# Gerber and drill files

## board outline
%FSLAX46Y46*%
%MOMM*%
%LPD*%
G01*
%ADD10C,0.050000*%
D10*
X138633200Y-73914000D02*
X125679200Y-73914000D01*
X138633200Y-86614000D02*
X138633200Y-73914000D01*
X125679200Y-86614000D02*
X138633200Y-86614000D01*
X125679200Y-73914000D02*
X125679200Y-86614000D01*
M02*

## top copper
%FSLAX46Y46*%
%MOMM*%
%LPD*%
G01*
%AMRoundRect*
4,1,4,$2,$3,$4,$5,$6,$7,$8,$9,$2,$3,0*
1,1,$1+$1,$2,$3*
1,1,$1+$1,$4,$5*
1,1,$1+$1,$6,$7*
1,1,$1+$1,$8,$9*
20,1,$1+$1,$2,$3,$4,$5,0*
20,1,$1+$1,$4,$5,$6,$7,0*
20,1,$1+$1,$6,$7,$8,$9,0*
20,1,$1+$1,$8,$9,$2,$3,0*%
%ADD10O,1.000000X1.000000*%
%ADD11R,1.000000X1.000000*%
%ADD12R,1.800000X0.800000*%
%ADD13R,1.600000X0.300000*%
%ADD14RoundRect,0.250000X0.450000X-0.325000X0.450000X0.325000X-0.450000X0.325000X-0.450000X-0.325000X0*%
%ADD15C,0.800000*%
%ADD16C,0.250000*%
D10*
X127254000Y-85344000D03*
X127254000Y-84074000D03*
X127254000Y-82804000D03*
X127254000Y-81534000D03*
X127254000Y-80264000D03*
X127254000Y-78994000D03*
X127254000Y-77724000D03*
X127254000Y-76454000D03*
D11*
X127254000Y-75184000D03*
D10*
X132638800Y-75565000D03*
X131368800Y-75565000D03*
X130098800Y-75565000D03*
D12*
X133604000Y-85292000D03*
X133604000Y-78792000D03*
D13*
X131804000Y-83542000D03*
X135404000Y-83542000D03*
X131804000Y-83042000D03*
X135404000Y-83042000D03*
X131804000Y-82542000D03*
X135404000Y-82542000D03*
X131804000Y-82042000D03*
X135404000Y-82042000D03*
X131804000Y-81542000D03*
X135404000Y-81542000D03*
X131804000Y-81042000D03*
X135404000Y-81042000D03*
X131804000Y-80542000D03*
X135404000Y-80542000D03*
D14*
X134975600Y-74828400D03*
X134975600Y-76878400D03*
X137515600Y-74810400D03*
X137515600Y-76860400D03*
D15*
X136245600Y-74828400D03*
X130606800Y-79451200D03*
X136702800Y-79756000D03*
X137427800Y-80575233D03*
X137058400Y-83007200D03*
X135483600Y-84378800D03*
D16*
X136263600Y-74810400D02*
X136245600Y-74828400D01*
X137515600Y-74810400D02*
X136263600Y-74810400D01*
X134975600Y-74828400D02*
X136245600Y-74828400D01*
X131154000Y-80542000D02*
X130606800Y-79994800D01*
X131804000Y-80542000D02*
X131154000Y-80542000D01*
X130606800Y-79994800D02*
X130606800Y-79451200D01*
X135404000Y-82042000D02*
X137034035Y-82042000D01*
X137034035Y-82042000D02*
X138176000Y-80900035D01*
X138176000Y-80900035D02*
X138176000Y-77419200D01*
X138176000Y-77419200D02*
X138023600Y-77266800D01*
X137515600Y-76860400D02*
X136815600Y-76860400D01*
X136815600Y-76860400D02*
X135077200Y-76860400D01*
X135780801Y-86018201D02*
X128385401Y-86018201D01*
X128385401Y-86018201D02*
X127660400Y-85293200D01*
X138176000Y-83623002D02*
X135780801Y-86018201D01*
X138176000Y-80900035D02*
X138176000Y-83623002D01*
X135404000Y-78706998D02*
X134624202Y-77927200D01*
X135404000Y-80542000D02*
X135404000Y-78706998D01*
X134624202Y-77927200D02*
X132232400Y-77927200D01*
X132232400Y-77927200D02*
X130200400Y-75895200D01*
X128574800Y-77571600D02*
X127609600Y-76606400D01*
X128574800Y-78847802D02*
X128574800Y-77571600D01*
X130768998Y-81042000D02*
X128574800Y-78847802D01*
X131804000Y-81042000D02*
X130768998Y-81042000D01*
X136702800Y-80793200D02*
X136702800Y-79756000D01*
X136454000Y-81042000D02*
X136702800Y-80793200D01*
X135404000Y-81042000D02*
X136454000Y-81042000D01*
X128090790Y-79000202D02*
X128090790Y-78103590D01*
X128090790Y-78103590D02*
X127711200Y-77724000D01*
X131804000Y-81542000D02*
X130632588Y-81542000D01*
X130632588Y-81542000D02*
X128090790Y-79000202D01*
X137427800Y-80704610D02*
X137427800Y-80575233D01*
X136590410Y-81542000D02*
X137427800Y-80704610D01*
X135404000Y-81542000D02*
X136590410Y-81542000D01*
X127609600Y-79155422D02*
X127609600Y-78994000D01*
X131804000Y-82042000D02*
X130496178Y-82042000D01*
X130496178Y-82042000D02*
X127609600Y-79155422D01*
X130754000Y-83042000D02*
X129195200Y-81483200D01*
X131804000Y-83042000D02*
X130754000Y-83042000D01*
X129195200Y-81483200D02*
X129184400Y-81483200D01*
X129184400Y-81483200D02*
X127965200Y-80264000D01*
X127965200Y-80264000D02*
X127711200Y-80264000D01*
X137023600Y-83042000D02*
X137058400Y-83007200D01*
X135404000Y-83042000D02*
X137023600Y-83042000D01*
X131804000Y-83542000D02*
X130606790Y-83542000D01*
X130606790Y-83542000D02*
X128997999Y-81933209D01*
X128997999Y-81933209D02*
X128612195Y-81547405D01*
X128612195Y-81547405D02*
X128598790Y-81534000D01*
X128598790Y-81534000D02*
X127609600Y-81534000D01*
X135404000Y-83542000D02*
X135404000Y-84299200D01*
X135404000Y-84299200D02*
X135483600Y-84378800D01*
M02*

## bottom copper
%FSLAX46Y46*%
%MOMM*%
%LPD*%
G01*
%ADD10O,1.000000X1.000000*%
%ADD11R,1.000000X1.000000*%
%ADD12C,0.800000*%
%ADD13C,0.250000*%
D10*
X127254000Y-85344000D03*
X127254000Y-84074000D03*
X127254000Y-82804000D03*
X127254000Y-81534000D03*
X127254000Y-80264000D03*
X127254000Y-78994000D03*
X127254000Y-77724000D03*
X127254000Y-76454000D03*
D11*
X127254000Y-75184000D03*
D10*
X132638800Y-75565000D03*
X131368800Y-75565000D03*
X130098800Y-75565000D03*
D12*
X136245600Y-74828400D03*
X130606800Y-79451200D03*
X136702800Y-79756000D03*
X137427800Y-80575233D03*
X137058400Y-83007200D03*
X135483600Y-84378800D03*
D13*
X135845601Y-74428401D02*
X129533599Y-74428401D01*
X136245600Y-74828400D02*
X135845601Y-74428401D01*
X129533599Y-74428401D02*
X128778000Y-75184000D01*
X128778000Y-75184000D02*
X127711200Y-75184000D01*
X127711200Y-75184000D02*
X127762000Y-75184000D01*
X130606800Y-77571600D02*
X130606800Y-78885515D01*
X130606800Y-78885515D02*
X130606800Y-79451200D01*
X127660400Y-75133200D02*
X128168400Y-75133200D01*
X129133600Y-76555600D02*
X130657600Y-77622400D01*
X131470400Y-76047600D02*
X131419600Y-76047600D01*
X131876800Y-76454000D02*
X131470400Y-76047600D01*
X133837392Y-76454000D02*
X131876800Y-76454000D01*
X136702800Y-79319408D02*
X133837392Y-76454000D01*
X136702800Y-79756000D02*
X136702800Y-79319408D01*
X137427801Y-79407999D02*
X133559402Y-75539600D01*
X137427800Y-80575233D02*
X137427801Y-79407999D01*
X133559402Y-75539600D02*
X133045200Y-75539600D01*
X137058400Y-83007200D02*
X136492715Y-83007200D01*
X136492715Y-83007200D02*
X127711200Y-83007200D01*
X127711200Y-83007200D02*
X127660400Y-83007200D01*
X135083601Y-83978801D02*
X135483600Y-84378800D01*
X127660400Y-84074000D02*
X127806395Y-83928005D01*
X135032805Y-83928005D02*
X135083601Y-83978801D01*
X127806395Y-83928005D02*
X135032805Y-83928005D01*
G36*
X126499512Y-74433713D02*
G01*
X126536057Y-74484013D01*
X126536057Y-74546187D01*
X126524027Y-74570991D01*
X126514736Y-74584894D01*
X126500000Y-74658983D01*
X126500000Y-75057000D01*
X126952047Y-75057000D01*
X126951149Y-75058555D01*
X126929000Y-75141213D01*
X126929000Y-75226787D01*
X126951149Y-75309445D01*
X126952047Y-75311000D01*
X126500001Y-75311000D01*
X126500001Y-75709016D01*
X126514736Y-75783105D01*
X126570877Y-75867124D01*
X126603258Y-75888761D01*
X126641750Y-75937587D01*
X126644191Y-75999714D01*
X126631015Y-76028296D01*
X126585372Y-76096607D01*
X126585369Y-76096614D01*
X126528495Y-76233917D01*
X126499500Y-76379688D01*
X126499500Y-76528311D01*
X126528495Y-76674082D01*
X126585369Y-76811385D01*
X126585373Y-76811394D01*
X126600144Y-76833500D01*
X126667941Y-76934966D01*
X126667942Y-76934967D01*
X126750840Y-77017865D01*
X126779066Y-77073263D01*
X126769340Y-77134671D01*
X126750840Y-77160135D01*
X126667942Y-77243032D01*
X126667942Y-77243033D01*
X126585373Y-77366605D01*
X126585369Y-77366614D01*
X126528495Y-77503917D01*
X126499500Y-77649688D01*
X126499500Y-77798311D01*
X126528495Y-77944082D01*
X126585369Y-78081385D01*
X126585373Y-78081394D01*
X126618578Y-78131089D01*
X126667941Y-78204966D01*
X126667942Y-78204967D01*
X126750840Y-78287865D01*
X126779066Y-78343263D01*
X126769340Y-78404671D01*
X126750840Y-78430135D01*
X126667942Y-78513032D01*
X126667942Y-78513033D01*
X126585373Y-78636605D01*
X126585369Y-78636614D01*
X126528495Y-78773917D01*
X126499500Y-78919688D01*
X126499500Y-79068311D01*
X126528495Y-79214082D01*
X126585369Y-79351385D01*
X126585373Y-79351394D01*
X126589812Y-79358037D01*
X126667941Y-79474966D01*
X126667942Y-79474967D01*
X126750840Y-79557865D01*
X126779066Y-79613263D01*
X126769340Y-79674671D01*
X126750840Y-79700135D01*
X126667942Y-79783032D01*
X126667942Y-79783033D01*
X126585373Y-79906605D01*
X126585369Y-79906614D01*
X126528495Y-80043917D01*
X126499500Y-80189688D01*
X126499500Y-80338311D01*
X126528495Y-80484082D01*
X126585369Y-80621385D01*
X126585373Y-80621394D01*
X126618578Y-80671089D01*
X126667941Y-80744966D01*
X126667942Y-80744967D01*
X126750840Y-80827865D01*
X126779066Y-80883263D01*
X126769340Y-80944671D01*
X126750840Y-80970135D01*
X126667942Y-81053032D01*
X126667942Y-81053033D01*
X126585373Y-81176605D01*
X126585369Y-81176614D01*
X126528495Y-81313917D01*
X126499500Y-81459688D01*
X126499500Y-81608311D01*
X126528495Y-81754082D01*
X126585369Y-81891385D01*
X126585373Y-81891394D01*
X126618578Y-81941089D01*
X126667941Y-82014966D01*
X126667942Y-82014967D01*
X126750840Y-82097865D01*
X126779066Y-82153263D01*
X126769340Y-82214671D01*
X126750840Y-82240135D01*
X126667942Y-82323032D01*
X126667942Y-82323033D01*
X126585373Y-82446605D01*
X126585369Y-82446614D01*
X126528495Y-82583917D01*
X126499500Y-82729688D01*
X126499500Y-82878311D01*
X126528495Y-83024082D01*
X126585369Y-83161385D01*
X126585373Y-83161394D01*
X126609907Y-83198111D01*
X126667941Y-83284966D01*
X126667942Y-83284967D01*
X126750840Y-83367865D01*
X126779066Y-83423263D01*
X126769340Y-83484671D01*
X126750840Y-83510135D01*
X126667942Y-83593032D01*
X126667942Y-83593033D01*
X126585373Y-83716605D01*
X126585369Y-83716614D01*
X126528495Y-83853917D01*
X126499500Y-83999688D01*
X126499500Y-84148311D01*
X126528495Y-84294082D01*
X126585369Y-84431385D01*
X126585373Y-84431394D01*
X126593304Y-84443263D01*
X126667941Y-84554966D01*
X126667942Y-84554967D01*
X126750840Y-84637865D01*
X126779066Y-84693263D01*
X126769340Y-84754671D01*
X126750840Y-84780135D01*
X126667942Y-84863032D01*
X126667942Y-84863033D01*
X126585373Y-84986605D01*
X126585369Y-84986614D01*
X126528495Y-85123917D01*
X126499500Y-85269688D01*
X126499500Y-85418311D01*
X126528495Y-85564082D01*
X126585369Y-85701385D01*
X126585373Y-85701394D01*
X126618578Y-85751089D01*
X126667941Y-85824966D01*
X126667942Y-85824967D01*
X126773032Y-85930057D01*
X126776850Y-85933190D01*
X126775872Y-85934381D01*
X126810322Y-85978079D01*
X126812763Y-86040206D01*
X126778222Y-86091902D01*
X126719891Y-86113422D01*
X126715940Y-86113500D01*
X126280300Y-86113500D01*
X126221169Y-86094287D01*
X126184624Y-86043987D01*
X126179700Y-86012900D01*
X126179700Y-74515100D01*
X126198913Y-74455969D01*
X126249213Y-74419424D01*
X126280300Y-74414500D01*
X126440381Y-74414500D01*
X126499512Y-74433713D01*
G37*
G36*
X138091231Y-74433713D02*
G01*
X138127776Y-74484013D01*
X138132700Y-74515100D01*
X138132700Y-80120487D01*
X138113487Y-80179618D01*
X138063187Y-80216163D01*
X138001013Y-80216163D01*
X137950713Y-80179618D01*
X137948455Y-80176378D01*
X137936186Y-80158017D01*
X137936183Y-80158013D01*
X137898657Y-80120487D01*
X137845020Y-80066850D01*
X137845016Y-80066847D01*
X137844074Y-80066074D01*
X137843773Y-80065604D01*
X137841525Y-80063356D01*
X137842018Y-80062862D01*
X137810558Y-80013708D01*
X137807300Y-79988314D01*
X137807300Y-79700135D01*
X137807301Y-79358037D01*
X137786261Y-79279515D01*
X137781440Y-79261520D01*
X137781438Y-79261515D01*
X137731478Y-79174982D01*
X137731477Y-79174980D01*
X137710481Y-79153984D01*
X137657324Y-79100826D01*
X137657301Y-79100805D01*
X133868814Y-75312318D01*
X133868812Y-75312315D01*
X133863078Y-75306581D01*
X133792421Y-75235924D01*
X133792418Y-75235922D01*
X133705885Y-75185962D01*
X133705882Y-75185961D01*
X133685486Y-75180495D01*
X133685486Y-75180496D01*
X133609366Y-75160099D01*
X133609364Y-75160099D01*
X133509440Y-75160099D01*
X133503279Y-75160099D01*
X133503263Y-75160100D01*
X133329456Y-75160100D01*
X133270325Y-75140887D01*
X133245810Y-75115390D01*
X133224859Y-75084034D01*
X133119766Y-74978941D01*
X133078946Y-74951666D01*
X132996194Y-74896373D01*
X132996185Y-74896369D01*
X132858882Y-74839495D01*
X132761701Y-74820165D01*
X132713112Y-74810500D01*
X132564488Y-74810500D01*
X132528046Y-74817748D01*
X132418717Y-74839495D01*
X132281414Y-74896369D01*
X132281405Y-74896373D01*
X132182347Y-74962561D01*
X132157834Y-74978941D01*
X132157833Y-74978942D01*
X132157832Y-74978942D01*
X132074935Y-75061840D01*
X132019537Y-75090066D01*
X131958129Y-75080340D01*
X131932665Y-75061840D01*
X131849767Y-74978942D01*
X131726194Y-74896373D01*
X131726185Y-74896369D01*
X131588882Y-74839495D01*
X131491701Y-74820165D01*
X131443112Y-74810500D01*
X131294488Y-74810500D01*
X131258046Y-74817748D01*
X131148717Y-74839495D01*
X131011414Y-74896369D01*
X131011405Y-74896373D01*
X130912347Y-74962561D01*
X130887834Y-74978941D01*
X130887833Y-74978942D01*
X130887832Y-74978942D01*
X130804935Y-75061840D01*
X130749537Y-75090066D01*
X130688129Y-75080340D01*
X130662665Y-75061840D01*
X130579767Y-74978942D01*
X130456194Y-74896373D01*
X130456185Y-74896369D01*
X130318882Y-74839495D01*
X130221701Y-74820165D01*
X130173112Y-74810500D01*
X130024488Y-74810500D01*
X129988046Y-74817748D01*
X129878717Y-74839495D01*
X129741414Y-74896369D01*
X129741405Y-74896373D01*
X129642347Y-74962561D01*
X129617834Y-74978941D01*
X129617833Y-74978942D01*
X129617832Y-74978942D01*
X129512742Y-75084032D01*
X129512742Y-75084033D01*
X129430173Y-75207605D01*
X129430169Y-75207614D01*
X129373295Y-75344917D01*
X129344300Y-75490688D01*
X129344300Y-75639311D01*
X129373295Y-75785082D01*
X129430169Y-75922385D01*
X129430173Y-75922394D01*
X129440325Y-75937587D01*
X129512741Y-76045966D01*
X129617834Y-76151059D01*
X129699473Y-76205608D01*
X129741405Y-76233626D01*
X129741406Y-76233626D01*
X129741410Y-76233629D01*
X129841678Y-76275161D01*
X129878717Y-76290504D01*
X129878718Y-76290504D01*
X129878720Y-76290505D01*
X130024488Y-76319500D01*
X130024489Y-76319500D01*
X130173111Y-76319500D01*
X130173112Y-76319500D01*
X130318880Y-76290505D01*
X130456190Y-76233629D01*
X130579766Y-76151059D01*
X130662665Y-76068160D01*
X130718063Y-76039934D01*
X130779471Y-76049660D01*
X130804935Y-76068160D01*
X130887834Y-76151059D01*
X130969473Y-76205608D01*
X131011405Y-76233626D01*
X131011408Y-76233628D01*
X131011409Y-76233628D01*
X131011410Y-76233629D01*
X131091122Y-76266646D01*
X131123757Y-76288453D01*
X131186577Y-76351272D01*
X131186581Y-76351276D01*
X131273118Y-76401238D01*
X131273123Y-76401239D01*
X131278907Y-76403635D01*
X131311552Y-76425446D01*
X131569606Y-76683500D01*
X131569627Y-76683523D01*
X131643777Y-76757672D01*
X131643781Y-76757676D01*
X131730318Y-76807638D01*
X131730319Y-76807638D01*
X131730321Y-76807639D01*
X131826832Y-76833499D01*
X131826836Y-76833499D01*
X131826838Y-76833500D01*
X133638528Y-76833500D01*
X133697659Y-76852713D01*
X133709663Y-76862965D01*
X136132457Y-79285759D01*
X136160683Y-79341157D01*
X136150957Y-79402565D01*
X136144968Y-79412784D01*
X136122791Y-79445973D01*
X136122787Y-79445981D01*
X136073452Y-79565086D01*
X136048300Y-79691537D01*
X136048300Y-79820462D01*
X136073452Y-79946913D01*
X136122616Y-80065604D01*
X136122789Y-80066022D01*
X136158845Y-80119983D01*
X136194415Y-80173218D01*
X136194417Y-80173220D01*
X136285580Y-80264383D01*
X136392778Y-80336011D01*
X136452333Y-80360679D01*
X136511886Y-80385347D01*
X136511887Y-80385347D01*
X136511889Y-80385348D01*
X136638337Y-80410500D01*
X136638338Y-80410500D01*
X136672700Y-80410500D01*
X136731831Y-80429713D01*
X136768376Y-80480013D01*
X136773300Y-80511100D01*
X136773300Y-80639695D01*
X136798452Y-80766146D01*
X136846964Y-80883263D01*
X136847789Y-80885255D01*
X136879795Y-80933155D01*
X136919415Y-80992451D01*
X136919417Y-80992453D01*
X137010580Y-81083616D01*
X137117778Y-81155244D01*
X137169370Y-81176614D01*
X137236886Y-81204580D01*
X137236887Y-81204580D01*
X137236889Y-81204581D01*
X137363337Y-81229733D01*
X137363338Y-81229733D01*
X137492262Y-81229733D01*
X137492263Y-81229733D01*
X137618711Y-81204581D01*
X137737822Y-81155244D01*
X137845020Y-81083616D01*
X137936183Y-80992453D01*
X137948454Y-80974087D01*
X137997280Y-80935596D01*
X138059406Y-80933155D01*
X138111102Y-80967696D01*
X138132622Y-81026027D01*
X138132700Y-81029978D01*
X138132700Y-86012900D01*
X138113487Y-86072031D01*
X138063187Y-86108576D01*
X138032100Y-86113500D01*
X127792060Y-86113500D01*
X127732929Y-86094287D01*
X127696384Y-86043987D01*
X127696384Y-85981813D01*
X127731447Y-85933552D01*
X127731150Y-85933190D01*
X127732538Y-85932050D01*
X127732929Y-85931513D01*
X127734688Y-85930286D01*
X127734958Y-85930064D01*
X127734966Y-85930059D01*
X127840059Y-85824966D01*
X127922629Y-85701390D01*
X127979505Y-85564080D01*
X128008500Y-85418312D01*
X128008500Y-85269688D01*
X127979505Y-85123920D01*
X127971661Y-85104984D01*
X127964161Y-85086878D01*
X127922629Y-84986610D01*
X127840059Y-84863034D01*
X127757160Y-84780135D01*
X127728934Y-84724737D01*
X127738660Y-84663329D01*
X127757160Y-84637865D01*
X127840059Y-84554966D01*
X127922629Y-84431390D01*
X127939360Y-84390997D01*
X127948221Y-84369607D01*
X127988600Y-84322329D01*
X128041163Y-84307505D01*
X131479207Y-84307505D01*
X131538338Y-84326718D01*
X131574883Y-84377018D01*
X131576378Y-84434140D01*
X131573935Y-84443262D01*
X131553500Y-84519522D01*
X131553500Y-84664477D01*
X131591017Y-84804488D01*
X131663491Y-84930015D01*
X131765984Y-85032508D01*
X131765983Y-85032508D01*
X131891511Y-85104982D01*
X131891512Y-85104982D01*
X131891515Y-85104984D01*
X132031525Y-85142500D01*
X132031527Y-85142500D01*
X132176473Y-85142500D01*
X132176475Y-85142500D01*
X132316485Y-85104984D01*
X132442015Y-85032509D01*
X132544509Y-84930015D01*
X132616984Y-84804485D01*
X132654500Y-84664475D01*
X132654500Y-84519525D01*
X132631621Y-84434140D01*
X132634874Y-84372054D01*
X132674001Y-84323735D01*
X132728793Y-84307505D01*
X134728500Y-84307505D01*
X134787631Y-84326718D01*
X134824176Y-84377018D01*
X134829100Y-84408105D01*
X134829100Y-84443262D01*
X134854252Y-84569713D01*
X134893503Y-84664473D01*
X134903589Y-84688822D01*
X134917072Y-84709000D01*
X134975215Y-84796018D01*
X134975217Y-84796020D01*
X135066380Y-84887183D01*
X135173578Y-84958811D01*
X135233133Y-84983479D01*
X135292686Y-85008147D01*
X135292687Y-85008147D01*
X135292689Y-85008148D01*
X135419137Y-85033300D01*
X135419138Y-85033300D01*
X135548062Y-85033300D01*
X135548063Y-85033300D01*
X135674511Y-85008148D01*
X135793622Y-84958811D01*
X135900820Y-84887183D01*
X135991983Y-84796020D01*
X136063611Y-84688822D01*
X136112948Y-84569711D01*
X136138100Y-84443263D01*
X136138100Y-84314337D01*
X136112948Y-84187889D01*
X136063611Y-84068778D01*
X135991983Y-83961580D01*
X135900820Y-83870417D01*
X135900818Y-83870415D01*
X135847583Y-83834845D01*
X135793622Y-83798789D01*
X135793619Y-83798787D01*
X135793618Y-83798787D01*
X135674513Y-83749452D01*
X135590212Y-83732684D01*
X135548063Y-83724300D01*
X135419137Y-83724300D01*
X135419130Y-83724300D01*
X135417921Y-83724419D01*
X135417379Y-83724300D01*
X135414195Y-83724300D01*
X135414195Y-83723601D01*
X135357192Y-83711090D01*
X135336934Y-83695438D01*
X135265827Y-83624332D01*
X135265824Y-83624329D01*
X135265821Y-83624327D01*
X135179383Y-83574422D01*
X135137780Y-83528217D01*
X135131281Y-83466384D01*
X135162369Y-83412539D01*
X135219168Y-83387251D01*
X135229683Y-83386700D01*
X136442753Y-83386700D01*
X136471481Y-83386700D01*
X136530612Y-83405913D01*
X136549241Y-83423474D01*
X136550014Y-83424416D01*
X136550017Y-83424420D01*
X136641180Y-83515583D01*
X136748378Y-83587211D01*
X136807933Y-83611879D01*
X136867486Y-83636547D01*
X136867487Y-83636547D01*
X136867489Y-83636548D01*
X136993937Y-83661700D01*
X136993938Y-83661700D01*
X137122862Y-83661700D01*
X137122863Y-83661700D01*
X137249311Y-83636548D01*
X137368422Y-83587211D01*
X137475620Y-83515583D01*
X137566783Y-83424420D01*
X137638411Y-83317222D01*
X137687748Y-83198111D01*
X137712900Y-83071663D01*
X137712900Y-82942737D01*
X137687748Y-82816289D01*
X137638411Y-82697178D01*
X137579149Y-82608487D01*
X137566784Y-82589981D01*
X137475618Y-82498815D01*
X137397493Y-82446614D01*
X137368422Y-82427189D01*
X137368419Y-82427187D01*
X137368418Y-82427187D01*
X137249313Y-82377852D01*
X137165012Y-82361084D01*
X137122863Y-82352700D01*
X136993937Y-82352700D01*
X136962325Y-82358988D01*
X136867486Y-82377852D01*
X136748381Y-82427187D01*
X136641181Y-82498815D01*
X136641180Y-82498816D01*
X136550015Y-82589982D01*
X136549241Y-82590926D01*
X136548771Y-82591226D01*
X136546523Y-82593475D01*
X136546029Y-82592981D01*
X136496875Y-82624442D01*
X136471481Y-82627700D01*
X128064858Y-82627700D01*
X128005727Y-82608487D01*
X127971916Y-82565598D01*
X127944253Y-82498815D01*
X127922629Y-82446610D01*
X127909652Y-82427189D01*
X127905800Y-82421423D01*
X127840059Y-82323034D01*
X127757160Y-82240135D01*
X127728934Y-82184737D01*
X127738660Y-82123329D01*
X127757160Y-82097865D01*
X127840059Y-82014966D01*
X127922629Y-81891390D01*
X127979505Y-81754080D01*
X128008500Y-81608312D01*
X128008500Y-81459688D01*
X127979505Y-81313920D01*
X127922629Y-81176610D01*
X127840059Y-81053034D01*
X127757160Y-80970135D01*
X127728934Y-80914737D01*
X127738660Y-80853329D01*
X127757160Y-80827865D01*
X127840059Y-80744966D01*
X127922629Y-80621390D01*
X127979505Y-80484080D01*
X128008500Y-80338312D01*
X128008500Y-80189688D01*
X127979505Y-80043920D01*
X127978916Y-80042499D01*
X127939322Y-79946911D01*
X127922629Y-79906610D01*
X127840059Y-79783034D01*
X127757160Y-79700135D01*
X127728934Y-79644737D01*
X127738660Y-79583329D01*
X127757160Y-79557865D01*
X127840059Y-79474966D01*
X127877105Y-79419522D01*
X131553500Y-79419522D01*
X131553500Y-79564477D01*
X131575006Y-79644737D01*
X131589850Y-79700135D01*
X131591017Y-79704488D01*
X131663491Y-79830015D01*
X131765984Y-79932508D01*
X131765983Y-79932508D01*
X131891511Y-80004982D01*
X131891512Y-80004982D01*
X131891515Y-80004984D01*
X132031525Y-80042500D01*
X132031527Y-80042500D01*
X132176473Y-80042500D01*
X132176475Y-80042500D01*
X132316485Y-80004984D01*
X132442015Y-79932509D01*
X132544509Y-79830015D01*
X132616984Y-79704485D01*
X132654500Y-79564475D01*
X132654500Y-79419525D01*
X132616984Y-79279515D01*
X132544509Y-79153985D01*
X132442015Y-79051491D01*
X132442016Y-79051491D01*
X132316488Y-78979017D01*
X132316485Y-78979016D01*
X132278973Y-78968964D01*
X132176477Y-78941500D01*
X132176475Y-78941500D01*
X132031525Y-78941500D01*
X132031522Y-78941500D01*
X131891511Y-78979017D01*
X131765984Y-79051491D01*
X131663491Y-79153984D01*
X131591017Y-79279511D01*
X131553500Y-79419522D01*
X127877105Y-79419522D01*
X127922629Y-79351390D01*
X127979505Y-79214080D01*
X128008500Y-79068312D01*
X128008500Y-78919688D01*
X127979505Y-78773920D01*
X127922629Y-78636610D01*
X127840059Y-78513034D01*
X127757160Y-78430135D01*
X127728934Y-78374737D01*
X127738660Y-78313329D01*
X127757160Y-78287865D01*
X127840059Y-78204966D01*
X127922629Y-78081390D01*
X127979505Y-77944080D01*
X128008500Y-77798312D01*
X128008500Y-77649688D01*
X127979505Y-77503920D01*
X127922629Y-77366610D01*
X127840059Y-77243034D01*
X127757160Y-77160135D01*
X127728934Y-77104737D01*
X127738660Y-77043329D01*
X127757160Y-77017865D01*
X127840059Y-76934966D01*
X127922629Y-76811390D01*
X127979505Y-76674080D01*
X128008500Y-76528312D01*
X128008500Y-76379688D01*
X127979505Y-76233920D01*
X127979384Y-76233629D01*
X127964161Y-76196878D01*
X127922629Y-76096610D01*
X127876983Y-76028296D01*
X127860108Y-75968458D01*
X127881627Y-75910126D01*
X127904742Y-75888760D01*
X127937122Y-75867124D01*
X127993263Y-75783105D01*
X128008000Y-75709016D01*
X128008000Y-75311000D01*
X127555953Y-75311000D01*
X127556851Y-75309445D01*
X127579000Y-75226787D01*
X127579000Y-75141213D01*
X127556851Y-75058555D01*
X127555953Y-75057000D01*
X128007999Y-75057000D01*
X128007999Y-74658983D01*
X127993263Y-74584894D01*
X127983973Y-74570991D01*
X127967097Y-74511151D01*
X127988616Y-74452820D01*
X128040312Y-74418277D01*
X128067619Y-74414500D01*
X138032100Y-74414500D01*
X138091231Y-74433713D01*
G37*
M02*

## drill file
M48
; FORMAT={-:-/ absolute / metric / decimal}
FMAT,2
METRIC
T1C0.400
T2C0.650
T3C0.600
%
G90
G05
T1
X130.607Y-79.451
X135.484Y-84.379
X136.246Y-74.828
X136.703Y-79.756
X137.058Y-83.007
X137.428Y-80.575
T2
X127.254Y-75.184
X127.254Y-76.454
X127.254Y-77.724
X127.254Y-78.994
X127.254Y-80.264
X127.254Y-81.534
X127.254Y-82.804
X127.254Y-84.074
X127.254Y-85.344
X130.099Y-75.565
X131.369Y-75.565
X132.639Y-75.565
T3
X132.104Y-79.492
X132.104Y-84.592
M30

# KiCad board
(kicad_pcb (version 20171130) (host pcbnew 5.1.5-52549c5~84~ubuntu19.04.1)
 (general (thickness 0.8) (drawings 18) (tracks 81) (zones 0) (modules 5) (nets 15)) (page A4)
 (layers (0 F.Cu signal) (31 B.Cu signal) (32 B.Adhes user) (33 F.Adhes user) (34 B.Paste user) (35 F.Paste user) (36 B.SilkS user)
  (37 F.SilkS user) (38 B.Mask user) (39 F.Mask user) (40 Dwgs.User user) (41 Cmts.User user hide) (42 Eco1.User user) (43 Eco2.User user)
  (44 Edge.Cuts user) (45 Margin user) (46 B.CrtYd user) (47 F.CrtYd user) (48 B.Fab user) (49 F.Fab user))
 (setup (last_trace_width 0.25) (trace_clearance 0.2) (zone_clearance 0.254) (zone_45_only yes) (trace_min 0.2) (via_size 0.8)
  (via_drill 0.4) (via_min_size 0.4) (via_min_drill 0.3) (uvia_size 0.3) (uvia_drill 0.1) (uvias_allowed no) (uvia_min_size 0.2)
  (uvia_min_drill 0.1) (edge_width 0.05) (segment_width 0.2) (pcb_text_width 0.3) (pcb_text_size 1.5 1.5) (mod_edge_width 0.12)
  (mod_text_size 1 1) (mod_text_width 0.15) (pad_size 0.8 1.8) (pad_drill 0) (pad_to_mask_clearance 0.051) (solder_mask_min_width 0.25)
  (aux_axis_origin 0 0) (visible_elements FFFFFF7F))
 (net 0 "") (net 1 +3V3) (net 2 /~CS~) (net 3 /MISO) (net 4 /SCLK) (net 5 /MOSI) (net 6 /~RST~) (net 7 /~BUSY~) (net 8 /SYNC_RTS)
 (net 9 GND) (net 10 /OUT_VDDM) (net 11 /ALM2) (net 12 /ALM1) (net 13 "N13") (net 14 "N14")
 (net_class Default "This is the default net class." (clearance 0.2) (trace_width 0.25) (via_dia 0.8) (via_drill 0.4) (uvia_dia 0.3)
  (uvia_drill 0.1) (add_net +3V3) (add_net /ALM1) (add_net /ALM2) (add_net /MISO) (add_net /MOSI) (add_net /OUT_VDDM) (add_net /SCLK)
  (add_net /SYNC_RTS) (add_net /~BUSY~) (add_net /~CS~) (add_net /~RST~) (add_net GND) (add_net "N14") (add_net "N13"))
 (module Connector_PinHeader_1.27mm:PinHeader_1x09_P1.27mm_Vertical (layer F.Cu) (at 127.254 75.184)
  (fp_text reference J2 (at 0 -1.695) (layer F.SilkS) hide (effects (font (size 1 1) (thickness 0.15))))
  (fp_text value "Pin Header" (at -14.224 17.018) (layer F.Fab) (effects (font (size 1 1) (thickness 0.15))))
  (pad 9 thru_hole oval (at 0 10.16) (size 1 1) (drill 0.65) (layers *.Cu *.Mask) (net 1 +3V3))
  (pad 8 thru_hole oval (at 0 8.89) (size 1 1) (drill 0.65) (layers *.Cu *.Mask) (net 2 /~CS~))
  (pad 7 thru_hole oval (at 0 7.62) (size 1 1) (drill 0.65) (layers *.Cu *.Mask) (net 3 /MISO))
  (pad 6 thru_hole oval (at 0 6.35) (size 1 1) (drill 0.65) (layers *.Cu *.Mask) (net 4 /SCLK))
  (pad 5 thru_hole oval (at 0 5.08) (size 1 1) (drill 0.65) (layers *.Cu *.Mask) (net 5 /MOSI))
  (pad 4 thru_hole oval (at 0 3.81) (size 1 1) (drill 0.65) (layers *.Cu *.Mask) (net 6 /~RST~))
  (pad 3 thru_hole oval (at 0 2.54) (size 1 1) (drill 0.65) (layers *.Cu *.Mask) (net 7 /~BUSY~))
  (pad 2 thru_hole oval (at 0 1.27) (size 1 1) (drill 0.65) (layers *.Cu *.Mask) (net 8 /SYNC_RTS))
  (pad 1 thru_hole rect (at 0 0) (size 1 1) (drill 0.65) (layers *.Cu *.Mask) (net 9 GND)))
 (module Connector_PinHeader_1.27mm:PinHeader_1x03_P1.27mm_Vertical (layer F.Cu) (at 130.0988 75.565 90)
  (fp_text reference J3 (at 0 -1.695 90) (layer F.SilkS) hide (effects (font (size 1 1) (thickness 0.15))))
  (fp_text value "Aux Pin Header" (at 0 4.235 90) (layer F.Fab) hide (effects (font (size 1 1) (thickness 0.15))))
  (pad 3 thru_hole oval (at 0 2.54 90) (size 1 1) (drill 0.65) (layers *.Cu *.Mask) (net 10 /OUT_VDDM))
  (pad 2 thru_hole oval (at 0 1.27 90) (size 1 1) (drill 0.65) (layers *.Cu *.Mask) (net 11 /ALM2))
  (pad 1 thru_hole oval (at 0 0 90) (size 1 1) (drill 0.65) (layers *.Cu *.Mask) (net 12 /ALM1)))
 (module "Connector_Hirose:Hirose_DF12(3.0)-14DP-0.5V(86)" (layer F.Cu) (at 133.604 82.042 90)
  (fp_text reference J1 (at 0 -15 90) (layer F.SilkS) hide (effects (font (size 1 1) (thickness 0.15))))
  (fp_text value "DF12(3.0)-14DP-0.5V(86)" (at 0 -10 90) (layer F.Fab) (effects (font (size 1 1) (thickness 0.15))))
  (pad "" np_thru_hole circle (at 2.55 -1.5 90) (size 0.6 0.6) (drill 0.6) (layers *.Cu *.Mask))
  (pad MP smd rect (at -3.25 0 90) (size 0.8 1.8) (layers F.Cu F.Paste F.Mask))
  (pad MP smd rect (at 3.25 0 90) (size 0.8 1.8) (layers F.Cu F.Paste F.Mask))
  (pad 13 smd rect (at -1.5 -1.8 90) (size 0.3 1.6) (layers F.Cu F.Paste F.Mask) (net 4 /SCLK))
  (pad 14 smd rect (at -1.5 1.8 90) (size 0.3 1.6) (layers F.Cu F.Paste F.Mask) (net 2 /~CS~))
  (pad 11 smd rect (at -1 -1.8 90) (size 0.3 1.6) (layers F.Cu F.Paste F.Mask) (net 5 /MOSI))
  (pad 12 smd rect (at -1 1.8 90) (size 0.3 1.6) (layers F.Cu F.Paste F.Mask) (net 3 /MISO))
  (pad 9 smd rect (at -0.5 -1.8 90) (size 0.3 1.6) (layers F.Cu F.Paste F.Mask) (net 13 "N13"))
  (pad 10 smd rect (at -0.5 1.8 90) (size 0.3 1.6) (layers F.Cu F.Paste F.Mask) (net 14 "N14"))
  (pad 7 smd rect (at 0 -1.8 90) (size 0.3 1.6) (layers F.Cu F.Paste F.Mask) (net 6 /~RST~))
  (pad 8 smd rect (at 0 1.8 90) (size 0.3 1.6) (layers F.Cu F.Paste F.Mask) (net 1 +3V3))
  (pad 5 smd rect (at 0.5 -1.8 90) (size 0.3 1.6) (layers F.Cu F.Paste F.Mask) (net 7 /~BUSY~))
  (pad 6 smd rect (at 0.5 1.8 90) (size 0.3 1.6) (layers F.Cu F.Paste F.Mask) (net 10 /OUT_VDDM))
  (pad 3 smd rect (at 1 -1.8 90) (size 0.3 1.6) (layers F.Cu F.Paste F.Mask) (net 8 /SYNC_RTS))
  (pad 4 smd rect (at 1 1.8 90) (size 0.3 1.6) (layers F.Cu F.Paste F.Mask) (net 11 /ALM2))
  (pad 1 smd rect (at 1.5 -1.8 90) (size 0.3 1.6) (layers F.Cu F.Paste F.Mask) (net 9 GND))
  (pad 2 smd rect (at 1.5 1.8 90) (size 0.3 1.6) (layers F.Cu F.Paste F.Mask) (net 12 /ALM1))
  (pad "" np_thru_hole circle (at -2.55 -1.5 90) (size 0.6 0.6) (drill 0.6) (layers *.Cu *.Mask)))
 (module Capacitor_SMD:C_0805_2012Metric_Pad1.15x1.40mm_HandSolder (layer F.Cu) (at 134.9756 75.8534 90)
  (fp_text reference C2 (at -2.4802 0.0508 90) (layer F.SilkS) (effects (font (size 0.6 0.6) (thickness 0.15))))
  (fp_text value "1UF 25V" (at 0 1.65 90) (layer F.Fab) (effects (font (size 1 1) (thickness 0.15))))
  (pad 2 smd roundrect (at 1.025 0 90) (size 1.15 1.4) (layers F.Cu F.Paste F.Mask) (roundrect_rratio 0.217391) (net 9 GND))
  (pad 1 smd roundrect (at -1.025 0 90) (size 1.15 1.4) (layers F.Cu F.Paste F.Mask) (roundrect_rratio 0.217391) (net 1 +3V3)))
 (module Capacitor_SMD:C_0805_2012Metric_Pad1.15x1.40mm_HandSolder (layer F.Cu) (at 137.5156 75.8354 90)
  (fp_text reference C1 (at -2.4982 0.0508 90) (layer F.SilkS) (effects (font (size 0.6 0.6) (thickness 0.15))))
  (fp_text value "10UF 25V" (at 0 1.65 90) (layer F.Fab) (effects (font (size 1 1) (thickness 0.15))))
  (pad 2 smd roundrect (at 1.025 0 90) (size 1.15 1.4) (layers F.Cu F.Paste F.Mask) (roundrect_rratio 0.217391) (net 9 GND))
  (pad 1 smd roundrect (at -1.025 0 90) (size 1.15 1.4) (layers F.Cu F.Paste F.Mask) (roundrect_rratio 0.217391) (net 1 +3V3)))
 (gr_line (start 138.6332 73.914) (end 125.6792 73.914) (layer Edge.Cuts) (width 0.05))
 (gr_line (start 138.6332 86.614) (end 138.6332 73.914) (layer Edge.Cuts) (width 0.05))
 (gr_line (start 125.6792 86.614) (end 138.6332 86.614) (layer Edge.Cuts) (width 0.05))
 (gr_line (start 125.6792 73.914) (end 125.6792 86.614) (layer Edge.Cuts) (width 0.05))
 (segment (start 136.2636 74.8104) (end 136.2456 74.8284) (width 0.25) (layer F.Cu) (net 9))
 (via (at 136.2456 74.8284) (size 0.8) (drill 0.4) (layers F.Cu B.Cu) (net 9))
 (segment (start 137.5156 74.8104) (end 136.2636 74.8104) (width 0.25) (layer F.Cu) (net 9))
 (segment (start 135.845601 74.428401) (end 129.533599 74.428401) (width 0.25) (layer B.Cu) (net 9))
 (segment (start 136.2456 74.8284) (end 135.845601 74.428401) (width 0.25) (layer B.Cu) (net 9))
 (segment (start 129.533599 74.428401) (end 128.778 75.184) (width 0.25) (layer B.Cu) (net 9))
 (segment (start 128.778 75.184) (end 127.7112 75.184) (width 0.25) (layer B.Cu) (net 9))
 (segment (start 127.7112 75.184) (end 127.762 75.184) (width 0.25) (layer B.Cu) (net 9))
 (segment (start 134.9756 74.8284) (end 136.2456 74.8284) (width 0.25) (layer F.Cu) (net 9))
 (via (at 130.6068 79.4512) (size 0.8) (drill 0.4) (layers F.Cu B.Cu) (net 9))
 (segment (start 131.154 80.542) (end 130.6068 79.9948) (width 0.25) (layer F.Cu) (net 9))
 (segment (start 131.804 80.542) (end 131.154 80.542) (width 0.25) (layer F.Cu) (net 9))
 (segment (start 130.6068 79.9948) (end 130.6068 79.4512) (width 0.25) (layer F.Cu) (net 9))
 (segment (start 130.6068 77.5716) (end 130.6068 78.885515) (width 0.25) (layer B.Cu) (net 9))
 (segment (start 130.6068 78.885515) (end 130.6068 79.4512) (width 0.25) (layer B.Cu) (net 9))
 (segment (start 127.6604 75.1332) (end 128.1684 75.1332) (width 0.25) (layer B.Cu) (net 9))
 (segment (start 129.1336 76.5556) (end 130.6576 77.6224) (width 0.25) (layer B.Cu) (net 9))
 (segment (start 135.404 82.042) (end 137.034035 82.042) (width 0.25) (layer F.Cu) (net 1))
 (segment (start 137.034035 82.042) (end 138.176 80.900035) (width 0.25) (layer F.Cu) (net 1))
 (segment (start 138.176 80.900035) (end 138.176 77.4192) (width 0.25) (layer F.Cu) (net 1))
 (segment (start 138.176 77.4192) (end 138.0236 77.2668) (width 0.25) (layer F.Cu) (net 1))
 (segment (start 137.5156 76.8604) (end 136.8156 76.8604) (width 0.25) (layer F.Cu) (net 1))
 (segment (start 136.8156 76.8604) (end 135.0772 76.8604) (width 0.25) (layer F.Cu) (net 1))
 (segment (start 135.780801 86.018201) (end 128.385401 86.018201) (width 0.25) (layer F.Cu) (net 1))
 (segment (start 128.385401 86.018201) (end 127.6604 85.2932) (width 0.25) (layer F.Cu) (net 1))
 (segment (start 138.176 83.623002) (end 135.780801 86.018201) (width 0.25) (layer F.Cu) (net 1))
 (segment (start 138.176 80.900035) (end 138.176 83.623002) (width 0.25) (layer F.Cu) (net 1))
 (segment (start 135.404 78.706998) (end 134.624202 77.9272) (width 0.25) (layer F.Cu) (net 12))
 (segment (start 135.404 80.542) (end 135.404 78.706998) (width 0.25) (layer F.Cu) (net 12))
 (segment (start 134.624202 77.9272) (end 132.2324 77.9272) (width 0.25) (layer F.Cu) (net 12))
 (segment (start 132.2324 77.9272) (end 130.2004 75.8952) (width 0.25) (layer F.Cu) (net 12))
 (segment (start 128.5748 77.5716) (end 127.6096 76.6064) (width 0.25) (layer F.Cu) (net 8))
 (segment (start 128.5748 78.847802) (end 128.5748 77.5716) (width 0.25) (layer F.Cu) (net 8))
 (segment (start 130.768998 81.042) (end 128.5748 78.847802) (width 0.25) (layer F.Cu) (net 8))
 (segment (start 131.804 81.042) (end 130.768998 81.042) (width 0.25) (layer F.Cu) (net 8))
 (segment (start 136.7028 80.7932) (end 136.7028 79.756) (width 0.25) (layer F.Cu) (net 11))
 (via (at 136.7028 79.756) (size 0.8) (drill 0.4) (layers F.Cu B.Cu) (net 11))
 (segment (start 136.454 81.042) (end 136.7028 80.7932) (width 0.25) (layer F.Cu) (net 11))
 (segment (start 135.404 81.042) (end 136.454 81.042) (width 0.25) (layer F.Cu) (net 11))
 (segment (start 131.4704 76.0476) (end 131.4196 76.0476) (width 0.25) (layer B.Cu) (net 11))
 (segment (start 131.8768 76.454) (end 131.4704 76.0476) (width 0.25) (layer B.Cu) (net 11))
 (segment (start 133.837392 76.454) (end 131.8768 76.454) (width 0.25) (layer B.Cu) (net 11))
 (segment (start 136.7028 79.319408) (end 133.837392 76.454) (width 0.25) (layer B.Cu) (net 11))
 (segment (start 136.7028 79.756) (end 136.7028 79.319408) (width 0.25) (layer B.Cu) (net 11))
 (segment (start 128.09079 79.000202) (end 128.09079 78.10359) (width 0.25) (layer F.Cu) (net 7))
 (segment (start 128.09079 78.10359) (end 127.7112 77.724) (width 0.25) (layer F.Cu) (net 7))
 (segment (start 131.804 81.542) (end 130.632588 81.542) (width 0.25) (layer F.Cu) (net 7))
 (segment (start 130.632588 81.542) (end 128.09079 79.000202) (width 0.25) (layer F.Cu) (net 7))
 (segment (start 137.4278 80.70461) (end 137.4278 80.575233) (width 0.25) (layer F.Cu) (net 10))
 (segment (start 136.59041 81.542) (end 137.4278 80.70461) (width 0.25) (layer F.Cu) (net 10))
 (via (at 137.4278 80.575233) (size 0.8) (drill 0.4) (layers F.Cu B.Cu) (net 10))
 (segment (start 135.404 81.542) (end 136.59041 81.542) (width 0.25) (layer F.Cu) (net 10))
 (segment (start 137.427801 79.407999) (end 133.559402 75.5396) (width 0.25) (layer B.Cu) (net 10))
 (segment (start 137.4278 80.575233) (end 137.427801 79.407999) (width 0.25) (layer B.Cu) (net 10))
 (segment (start 133.559402 75.5396) (end 133.0452 75.5396) (width 0.25) (layer B.Cu) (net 10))
 (segment (start 127.6096 79.155422) (end 127.6096 78.994) (width 0.25) (layer F.Cu) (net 6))
 (segment (start 131.804 82.042) (end 130.496178 82.042) (width 0.25) (layer F.Cu) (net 6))
 (segment (start 130.496178 82.042) (end 127.6096 79.155422) (width 0.25) (layer F.Cu) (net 6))
 (segment (start 130.754 83.042) (end 129.1952 81.4832) (width 0.25) (layer F.Cu) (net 5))
 (segment (start 131.804 83.042) (end 130.754 83.042) (width 0.25) (layer F.Cu) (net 5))
 (segment (start 129.1952 81.4832) (end 129.1844 81.4832) (width 0.25) (layer F.Cu) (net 5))
 (segment (start 129.1844 81.4832) (end 127.9652 80.264) (width 0.25) (layer F.Cu) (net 5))
 (segment (start 127.9652 80.264) (end 127.7112 80.264) (width 0.25) (layer F.Cu) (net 5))
 (via (at 137.0584 83.0072) (size 0.8) (drill 0.4) (layers F.Cu B.Cu) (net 3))
 (segment (start 137.0236 83.042) (end 137.0584 83.0072) (width 0.25) (layer F.Cu) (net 3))
 (segment (start 135.404 83.042) (end 137.0236 83.042) (width 0.25) (layer F.Cu) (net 3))
 (segment (start 137.0584 83.0072) (end 136.492715 83.0072) (width 0.25) (layer B.Cu) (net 3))
 (segment (start 136.492715 83.0072) (end 127.7112 83.0072) (width 0.25) (layer B.Cu) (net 3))
 (segment (start 127.7112 83.0072) (end 127.6604 83.0072) (width 0.25) (layer B.Cu) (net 3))
 (segment (start 131.804 83.542) (end 130.60679 83.542) (width 0.25) (layer F.Cu) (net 4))
 (segment (start 130.60679 83.542) (end 128.997999 81.933209) (width 0.25) (layer F.Cu) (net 4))
 (segment (start 128.997999 81.933209) (end 128.612195 81.547405) (width 0.25) (layer F.Cu) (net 4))
 (segment (start 128.612195 81.547405) (end 128.59879 81.534) (width 0.25) (layer F.Cu) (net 4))
 (segment (start 128.59879 81.534) (end 127.6096 81.534) (width 0.25) (layer F.Cu) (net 4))
 (segment (start 135.083601 83.978801) (end 135.4836 84.3788) (width 0.25) (layer B.Cu) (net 2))
 (segment (start 135.404 83.542) (end 135.404 84.2992) (width 0.25) (layer F.Cu) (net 2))
 (segment (start 127.6604 84.074) (end 127.806395 83.928005) (width 0.25) (layer B.Cu) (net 2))
 (segment (start 135.032805 83.928005) (end 135.083601 83.978801) (width 0.25) (layer B.Cu) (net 2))
 (segment (start 127.806395 83.928005) (end 135.032805 83.928005) (width 0.25) (layer B.Cu) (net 2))
 (segment (start 135.404 84.2992) (end 135.4836 84.3788) (width 0.25) (layer F.Cu) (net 2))
 (via (at 135.4836 84.3788) (size 0.8) (drill 0.4) (layers F.Cu B.Cu) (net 2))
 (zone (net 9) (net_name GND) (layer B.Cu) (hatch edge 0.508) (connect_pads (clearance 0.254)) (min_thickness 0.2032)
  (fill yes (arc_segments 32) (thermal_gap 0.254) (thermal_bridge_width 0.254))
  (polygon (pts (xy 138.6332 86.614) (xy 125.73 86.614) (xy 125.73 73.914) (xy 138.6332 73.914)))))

